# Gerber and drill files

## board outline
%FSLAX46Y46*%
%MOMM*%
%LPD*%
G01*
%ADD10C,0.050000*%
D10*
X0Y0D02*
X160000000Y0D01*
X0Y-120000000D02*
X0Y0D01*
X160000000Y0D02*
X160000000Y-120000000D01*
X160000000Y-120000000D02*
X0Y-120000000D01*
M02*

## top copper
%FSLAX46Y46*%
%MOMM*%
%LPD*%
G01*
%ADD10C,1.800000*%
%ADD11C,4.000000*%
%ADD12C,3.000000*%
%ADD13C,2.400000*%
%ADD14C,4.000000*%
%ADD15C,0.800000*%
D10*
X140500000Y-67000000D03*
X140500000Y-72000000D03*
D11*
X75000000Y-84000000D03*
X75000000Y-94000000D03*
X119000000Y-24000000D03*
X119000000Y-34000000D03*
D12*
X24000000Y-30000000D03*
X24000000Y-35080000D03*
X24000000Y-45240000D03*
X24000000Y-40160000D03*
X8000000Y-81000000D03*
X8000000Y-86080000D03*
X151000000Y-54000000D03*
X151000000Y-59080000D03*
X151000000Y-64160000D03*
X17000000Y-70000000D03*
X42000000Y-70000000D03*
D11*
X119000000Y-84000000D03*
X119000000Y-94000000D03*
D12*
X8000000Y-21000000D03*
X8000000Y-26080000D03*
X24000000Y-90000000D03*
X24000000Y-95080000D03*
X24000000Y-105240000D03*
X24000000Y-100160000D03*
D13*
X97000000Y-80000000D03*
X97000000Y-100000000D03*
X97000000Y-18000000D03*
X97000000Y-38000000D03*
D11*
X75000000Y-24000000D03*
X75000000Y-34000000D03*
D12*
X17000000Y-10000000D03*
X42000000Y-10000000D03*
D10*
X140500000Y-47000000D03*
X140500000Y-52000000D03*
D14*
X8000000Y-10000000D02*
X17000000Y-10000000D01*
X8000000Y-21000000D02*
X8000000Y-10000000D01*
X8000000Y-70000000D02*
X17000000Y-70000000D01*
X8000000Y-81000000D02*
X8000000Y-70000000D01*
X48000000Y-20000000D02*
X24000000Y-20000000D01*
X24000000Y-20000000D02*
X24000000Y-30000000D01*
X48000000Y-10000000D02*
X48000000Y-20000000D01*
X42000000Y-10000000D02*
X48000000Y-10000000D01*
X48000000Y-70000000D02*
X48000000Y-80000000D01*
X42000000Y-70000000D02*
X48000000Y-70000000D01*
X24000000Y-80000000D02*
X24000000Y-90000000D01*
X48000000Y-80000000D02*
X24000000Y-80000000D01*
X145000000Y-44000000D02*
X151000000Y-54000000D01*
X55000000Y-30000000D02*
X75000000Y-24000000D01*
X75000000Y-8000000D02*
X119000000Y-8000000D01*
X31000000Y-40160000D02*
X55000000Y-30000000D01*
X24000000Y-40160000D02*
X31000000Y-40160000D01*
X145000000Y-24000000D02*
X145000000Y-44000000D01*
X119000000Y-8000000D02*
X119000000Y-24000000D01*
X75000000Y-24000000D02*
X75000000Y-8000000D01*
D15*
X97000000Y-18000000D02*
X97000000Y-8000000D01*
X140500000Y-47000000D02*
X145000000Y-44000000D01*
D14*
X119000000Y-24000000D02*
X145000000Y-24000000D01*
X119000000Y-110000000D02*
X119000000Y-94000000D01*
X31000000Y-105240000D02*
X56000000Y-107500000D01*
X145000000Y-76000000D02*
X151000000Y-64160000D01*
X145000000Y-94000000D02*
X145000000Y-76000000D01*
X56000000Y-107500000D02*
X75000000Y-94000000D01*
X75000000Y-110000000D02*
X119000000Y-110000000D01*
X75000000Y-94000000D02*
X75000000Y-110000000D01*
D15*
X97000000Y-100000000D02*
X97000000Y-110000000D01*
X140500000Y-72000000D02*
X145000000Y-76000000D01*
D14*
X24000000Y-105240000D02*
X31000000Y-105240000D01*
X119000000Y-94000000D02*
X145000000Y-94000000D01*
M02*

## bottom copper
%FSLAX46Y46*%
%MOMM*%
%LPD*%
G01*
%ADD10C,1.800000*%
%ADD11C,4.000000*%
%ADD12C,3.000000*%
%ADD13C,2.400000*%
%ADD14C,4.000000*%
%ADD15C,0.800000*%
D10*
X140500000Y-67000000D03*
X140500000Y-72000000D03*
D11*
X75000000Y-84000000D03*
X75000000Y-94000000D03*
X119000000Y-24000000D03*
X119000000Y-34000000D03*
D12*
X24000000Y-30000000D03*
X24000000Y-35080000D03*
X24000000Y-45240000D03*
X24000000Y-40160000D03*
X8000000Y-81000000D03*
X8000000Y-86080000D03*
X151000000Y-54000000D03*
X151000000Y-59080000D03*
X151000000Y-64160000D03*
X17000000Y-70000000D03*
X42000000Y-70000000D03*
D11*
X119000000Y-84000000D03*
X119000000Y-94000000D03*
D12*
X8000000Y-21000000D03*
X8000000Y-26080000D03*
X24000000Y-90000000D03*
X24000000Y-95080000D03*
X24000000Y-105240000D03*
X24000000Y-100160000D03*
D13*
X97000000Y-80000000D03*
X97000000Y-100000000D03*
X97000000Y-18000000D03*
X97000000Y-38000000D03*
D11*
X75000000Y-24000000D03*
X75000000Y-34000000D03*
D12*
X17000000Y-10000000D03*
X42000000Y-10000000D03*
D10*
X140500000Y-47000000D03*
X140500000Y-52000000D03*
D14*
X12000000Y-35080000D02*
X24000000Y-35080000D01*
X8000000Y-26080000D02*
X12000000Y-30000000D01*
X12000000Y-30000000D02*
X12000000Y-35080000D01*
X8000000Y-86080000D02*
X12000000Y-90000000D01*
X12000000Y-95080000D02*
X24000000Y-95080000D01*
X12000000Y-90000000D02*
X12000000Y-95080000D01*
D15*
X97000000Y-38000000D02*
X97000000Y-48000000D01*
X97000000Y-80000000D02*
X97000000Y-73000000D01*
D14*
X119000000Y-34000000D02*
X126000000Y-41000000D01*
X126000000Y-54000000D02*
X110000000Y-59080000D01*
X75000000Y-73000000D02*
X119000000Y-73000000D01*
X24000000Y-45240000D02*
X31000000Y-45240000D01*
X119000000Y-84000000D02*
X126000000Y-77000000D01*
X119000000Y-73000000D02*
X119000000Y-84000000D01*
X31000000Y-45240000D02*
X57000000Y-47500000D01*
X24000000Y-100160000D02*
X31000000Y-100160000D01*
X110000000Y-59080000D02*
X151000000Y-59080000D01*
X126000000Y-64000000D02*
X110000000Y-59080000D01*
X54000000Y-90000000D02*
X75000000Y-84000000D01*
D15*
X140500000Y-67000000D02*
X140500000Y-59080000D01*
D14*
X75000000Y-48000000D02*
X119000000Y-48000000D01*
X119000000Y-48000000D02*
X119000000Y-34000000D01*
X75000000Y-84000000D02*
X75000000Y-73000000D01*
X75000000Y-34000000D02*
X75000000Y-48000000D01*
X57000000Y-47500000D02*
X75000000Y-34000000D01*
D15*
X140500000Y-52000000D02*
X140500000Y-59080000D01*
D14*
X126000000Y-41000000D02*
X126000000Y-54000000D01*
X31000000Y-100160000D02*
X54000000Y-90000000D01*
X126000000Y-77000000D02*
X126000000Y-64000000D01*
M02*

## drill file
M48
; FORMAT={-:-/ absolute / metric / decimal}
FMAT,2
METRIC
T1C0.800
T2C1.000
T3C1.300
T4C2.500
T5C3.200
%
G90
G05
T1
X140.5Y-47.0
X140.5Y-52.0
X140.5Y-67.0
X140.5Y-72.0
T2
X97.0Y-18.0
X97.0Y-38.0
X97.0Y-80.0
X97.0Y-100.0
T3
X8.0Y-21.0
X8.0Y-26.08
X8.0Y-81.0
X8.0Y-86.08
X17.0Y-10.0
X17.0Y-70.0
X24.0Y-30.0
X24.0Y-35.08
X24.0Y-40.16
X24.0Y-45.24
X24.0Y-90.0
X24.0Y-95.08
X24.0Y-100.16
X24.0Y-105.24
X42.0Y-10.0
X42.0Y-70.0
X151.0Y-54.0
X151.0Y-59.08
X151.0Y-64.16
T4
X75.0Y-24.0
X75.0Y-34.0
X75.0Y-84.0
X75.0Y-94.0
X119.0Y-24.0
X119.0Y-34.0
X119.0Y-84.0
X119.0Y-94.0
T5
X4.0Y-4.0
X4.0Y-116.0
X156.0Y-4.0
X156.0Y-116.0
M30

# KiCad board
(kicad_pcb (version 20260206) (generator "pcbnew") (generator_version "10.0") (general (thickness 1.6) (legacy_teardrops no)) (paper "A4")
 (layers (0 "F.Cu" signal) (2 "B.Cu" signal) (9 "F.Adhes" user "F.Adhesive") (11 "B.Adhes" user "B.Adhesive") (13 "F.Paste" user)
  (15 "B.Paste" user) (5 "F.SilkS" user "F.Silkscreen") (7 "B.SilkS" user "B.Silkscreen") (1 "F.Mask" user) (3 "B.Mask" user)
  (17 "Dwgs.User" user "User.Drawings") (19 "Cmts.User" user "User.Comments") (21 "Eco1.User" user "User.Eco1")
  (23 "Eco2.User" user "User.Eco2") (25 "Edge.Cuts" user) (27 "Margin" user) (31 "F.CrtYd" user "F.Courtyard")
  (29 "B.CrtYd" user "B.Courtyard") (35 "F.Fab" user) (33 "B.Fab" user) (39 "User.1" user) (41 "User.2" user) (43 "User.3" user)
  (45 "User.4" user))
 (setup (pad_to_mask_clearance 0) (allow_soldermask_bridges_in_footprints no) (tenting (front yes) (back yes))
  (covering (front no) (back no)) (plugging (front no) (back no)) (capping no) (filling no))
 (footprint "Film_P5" (layer "F.Cu") (at 140.5 67 -90)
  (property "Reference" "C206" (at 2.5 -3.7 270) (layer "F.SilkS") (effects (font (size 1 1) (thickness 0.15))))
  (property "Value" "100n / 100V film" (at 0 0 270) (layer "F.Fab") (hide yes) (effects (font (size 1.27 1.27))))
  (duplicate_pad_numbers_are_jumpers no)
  (pad "1" thru_hole circle (at 0 0 270) (size 1.8 1.8) (drill 0.8) (layers "*.Cu" "*.Mask") (remove_unused_layers no) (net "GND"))
  (pad "2" thru_hole circle (at 5 0 270) (size 1.8 1.8) (drill 0.8) (layers "*.Cu" "*.Mask") (remove_unused_layers no) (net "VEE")))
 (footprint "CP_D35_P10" (layer "F.Cu") (at 75 84 -90)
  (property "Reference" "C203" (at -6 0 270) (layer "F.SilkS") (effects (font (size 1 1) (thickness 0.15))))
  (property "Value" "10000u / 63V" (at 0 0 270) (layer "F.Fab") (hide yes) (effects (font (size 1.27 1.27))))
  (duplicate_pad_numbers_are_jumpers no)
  (pad "1" thru_hole circle (at 0 0 270) (size 4 4) (drill 2.5) (layers "*.Cu" "*.Mask") (remove_unused_layers no) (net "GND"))
  (pad "2" thru_hole circle (at 10 0 270) (size 4 4) (drill 2.5) (layers "*.Cu" "*.Mask") (remove_unused_layers no) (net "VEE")))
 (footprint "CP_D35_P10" (layer "F.Cu") (at 119 24 -90)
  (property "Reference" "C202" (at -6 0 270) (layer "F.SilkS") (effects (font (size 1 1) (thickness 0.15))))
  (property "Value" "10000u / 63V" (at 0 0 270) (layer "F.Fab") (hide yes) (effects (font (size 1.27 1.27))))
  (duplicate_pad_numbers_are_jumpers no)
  (pad "1" thru_hole circle (at 0 0 270) (size 4 4) (drill 2.5) (layers "*.Cu" "*.Mask") (remove_unused_layers no) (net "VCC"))
  (pad "2" thru_hole circle (at 10 0 270) (size 4 4) (drill 2.5) (layers "*.Cu" "*.Mask") (remove_unused_layers no) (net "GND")))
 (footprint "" (layer "F.Cu") (at 156 116)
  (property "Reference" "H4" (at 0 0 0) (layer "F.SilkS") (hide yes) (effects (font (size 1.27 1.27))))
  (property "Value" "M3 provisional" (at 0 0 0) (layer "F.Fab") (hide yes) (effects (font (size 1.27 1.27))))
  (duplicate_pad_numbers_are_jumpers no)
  (pad "" np_thru_hole circle (at 0 0) (size 3.2 3.2) (drill 3.2) (layers "*.Cu" "*.Mask")))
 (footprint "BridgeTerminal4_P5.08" (layer "F.Cu") (at 24 30 -90)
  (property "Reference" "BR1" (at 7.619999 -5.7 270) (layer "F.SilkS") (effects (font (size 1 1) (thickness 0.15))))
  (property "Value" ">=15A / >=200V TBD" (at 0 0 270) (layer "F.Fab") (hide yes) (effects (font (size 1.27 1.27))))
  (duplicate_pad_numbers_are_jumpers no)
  (pad "AC1" thru_hole circle (at 0 0 270) (size 3 3) (drill 1.3) (layers "*.Cu" "*.Mask") (remove_unused_layers no) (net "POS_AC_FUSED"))
  (pad "AC2" thru_hole circle (at 5.08 0 270) (size 3 3) (drill 1.3) (layers "*.Cu" "*.Mask") (remove_unused_layers no) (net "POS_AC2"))
  (pad "N" thru_hole circle (at 15.24 0 270) (size 3 3) (drill 1.3) (layers "*.Cu" "*.Mask") (remove_unused_layers no) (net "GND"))
  (pad "P" thru_hole circle (at 10.16 0 270) (size 3 3) (drill 1.3) (layers "*.Cu" "*.Mask") (remove_unused_layers no) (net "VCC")))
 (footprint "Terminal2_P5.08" (layer "F.Cu") (at 8 81 -90)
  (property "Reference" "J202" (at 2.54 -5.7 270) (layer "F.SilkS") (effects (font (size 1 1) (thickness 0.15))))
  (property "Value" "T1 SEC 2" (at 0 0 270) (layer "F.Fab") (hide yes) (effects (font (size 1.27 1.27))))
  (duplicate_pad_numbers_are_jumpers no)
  (pad "1" thru_hole circle (at 0 0 270) (size 3 3) (drill 1.3) (layers "*.Cu" "*.Mask") (remove_unused_layers no) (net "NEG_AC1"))
  (pad "2" thru_hole circle (at 5.08 0 270) (size 3 3) (drill 1.3) (layers "*.Cu" "*.Mask") (remove_unused_layers no) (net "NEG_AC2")))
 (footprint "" (layer "F.Cu") (at 4 4)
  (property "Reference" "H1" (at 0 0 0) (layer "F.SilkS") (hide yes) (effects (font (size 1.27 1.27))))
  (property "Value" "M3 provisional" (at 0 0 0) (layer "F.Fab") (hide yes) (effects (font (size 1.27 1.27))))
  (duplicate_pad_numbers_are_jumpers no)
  (pad "" np_thru_hole circle (at 0 0) (size 3.2 3.2) (drill 3.2) (layers "*.Cu" "*.Mask")))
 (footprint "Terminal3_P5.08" (layer "F.Cu") (at 151 54 -90)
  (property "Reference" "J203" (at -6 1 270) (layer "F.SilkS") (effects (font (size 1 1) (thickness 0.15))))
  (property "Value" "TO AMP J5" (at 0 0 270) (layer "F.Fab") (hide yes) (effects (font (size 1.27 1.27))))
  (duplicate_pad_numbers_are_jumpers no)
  (pad "1" thru_hole circle (at 0 0 270) (size 3 3) (drill 1.3) (layers "*.Cu" "*.Mask") (remove_unused_layers no) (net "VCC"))
  (pad "2" thru_hole circle (at 5.08 0 270) (size 3 3) (drill 1.3) (layers "*.Cu" "*.Mask") (remove_unused_layers no) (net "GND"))
  (pad "3" thru_hole circle (at 10.16 0 270) (size 3 3) (drill 1.3) (layers "*.Cu" "*.Mask") (remove_unused_layers no) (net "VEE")))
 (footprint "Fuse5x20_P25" (layer "F.Cu") (at 17 70)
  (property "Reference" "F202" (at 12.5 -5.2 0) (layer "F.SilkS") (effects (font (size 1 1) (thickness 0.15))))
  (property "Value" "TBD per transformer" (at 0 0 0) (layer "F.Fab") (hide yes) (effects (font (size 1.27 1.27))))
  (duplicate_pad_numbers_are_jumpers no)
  (pad "1" thru_hole circle (at 0 0) (size 3 3) (drill 1.3) (layers "*.Cu" "*.Mask") (remove_unused_layers no) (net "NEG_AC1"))
  (pad "2" thru_hole circle (at 25 0) (size 3 3) (drill 1.3) (layers "*.Cu" "*.Mask") (remove_unused_layers no) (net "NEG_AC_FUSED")))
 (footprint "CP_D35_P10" (layer "F.Cu") (at 119 84 -90)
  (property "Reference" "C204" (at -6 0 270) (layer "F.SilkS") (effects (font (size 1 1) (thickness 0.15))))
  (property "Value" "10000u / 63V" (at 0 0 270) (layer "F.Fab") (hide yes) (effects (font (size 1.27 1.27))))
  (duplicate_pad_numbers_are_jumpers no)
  (pad "1" thru_hole circle (at 0 0 270) (size 4 4) (drill 2.5) (layers "*.Cu" "*.Mask") (remove_unused_layers no) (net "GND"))
  (pad "2" thru_hole circle (at 10 0 270) (size 4 4) (drill 2.5) (layers "*.Cu" "*.Mask") (remove_unused_layers no) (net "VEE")))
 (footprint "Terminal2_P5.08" (layer "F.Cu") (at 8 21 -90)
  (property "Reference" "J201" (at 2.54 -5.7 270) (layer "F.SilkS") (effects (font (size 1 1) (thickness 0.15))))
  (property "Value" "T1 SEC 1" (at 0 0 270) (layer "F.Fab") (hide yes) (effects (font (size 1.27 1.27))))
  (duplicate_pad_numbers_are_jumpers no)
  (pad "1" thru_hole circle (at 0 0 270) (size 3 3) (drill 1.3) (layers "*.Cu" "*.Mask") (remove_unused_layers no) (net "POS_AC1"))
  (pad "2" thru_hole circle (at 5.08 0 270) (size 3 3) (drill 1.3) (layers "*.Cu" "*.Mask") (remove_unused_layers no) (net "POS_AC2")))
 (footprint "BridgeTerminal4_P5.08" (layer "F.Cu") (at 24 90 -90)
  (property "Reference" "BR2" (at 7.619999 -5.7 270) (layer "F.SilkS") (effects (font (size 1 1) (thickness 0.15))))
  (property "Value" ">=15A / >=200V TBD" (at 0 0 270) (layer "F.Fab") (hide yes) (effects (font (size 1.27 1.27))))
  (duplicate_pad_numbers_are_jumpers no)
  (pad "AC1" thru_hole circle (at 0 0 270) (size 3 3) (drill 1.3) (layers "*.Cu" "*.Mask") (remove_unused_layers no) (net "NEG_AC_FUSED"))
  (pad "AC2" thru_hole circle (at 5.08 0 270) (size 3 3) (drill 1.3) (layers "*.Cu" "*.Mask") (remove_unused_layers no) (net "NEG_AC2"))
  (pad "N" thru_hole circle (at 15.24 0 270) (size 3 3) (drill 1.3) (layers "*.Cu" "*.Mask") (remove_unused_layers no) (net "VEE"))
  (pad "P" thru_hole circle (at 10.16 0 270) (size 3 3) (drill 1.3) (layers "*.Cu" "*.Mask") (remove_unused_layers no) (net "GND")))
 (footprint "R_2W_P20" (layer "F.Cu") (at 97 80 -90)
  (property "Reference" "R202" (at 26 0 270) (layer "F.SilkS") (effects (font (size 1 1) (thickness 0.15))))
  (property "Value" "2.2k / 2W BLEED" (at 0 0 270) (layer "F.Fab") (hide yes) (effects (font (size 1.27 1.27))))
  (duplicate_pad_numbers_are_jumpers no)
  (pad "1" thru_hole circle (at 0 0 270) (size 2.4 2.4) (drill 1) (layers "*.Cu" "*.Mask") (remove_unused_layers no) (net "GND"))
  (pad "2" thru_hole circle (at 20 0 270) (size 2.4 2.4) (drill 1) (layers "*.Cu" "*.Mask") (remove_unused_layers no) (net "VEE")))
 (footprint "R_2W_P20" (layer "F.Cu") (at 97 18 -90)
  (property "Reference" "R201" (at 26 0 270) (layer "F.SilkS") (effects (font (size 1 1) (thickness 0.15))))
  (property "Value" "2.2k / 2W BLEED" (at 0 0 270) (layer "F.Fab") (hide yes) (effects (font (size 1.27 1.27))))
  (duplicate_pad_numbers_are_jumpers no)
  (pad "1" thru_hole circle (at 0 0 270) (size 2.4 2.4) (drill 1) (layers "*.Cu" "*.Mask") (remove_unused_layers no) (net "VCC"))
  (pad "2" thru_hole circle (at 20 0 270) (size 2.4 2.4) (drill 1) (layers "*.Cu" "*.Mask") (remove_unused_layers no) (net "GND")))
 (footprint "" (layer "F.Cu") (at 156 4)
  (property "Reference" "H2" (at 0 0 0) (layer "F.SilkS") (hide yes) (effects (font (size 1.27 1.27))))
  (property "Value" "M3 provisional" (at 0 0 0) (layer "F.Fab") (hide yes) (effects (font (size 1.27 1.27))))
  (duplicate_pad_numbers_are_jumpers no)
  (pad "" np_thru_hole circle (at 0 0) (size 3.2 3.2) (drill 3.2) (layers "*.Cu" "*.Mask")))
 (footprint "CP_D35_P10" (layer "F.Cu") (at 75 24 -90)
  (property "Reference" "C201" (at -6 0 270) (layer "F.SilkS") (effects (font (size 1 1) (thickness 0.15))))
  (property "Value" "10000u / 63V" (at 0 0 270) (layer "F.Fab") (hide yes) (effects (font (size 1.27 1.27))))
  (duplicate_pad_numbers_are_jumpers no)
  (pad "1" thru_hole circle (at 0 0 270) (size 4 4) (drill 2.5) (layers "*.Cu" "*.Mask") (remove_unused_layers no) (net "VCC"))
  (pad "2" thru_hole circle (at 10 0 270) (size 4 4) (drill 2.5) (layers "*.Cu" "*.Mask") (remove_unused_layers no) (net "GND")))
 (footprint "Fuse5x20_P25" (layer "F.Cu") (at 17 10)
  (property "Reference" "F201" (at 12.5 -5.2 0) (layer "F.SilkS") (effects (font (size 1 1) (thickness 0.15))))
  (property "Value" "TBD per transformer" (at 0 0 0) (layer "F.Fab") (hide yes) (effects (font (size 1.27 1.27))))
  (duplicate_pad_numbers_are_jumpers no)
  (pad "1" thru_hole circle (at 0 0) (size 3 3) (drill 1.3) (layers "*.Cu" "*.Mask") (remove_unused_layers no) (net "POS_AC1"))
  (pad "2" thru_hole circle (at 25 0) (size 3 3) (drill 1.3) (layers "*.Cu" "*.Mask") (remove_unused_layers no) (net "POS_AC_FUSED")))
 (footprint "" (layer "F.Cu") (at 4 116)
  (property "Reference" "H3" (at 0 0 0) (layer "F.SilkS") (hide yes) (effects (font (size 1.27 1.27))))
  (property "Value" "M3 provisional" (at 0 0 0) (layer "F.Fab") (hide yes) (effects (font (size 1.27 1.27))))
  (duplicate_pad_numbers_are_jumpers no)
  (pad "" np_thru_hole circle (at 0 0) (size 3.2 3.2) (drill 3.2) (layers "*.Cu" "*.Mask")))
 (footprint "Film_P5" (layer "F.Cu") (at 140.5 47 -90)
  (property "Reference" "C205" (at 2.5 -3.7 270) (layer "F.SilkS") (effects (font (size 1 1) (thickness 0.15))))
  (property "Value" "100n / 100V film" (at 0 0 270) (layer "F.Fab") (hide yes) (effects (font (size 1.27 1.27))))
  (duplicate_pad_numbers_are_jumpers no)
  (pad "1" thru_hole circle (at 0 0 270) (size 1.8 1.8) (drill 0.8) (layers "*.Cu" "*.Mask") (remove_unused_layers no) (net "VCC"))
  (pad "2" thru_hole circle (at 5 0 270) (size 1.8 1.8) (drill 0.8) (layers "*.Cu" "*.Mask") (remove_unused_layers no) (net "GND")))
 (gr_line (start 0 0) (end 160 0) (stroke (width 0.05) (type default)) (layer "Edge.Cuts"))
 (gr_line (start 0 120) (end 0 0) (stroke (width 0.05) (type default)) (layer "Edge.Cuts"))
 (gr_line (start 160 0) (end 160 120) (stroke (width 0.05) (type default)) (layer "Edge.Cuts"))
 (gr_line (start 160 120) (end 0 120) (stroke (width 0.05) (type default)) (layer "Edge.Cuts"))
 (segment (start 8 10) (end 17 10) (width 4) (layer "F.Cu") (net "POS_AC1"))
 (segment (start 8 21) (end 8 10) (width 4) (layer "F.Cu") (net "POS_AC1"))
 (segment (start 12 35.08) (end 24 35.08) (width 4) (layer "B.Cu") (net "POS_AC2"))
 (segment (start 8 26.08) (end 12 30) (width 4) (layer "B.Cu") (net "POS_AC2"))
 (segment (start 12 30) (end 12 35.08) (width 4) (layer "B.Cu") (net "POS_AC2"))
 (segment (start 8 70) (end 17 70) (width 4) (layer "F.Cu") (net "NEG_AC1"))
 (segment (start 8 81) (end 8 70) (width 4) (layer "F.Cu") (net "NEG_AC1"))
 (segment (start 8 86.08) (end 12 90) (width 4) (layer "B.Cu") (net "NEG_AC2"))
 (segment (start 12 95.08) (end 24 95.08) (width 4) (layer "B.Cu") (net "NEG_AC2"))
 (segment (start 12 90) (end 12 95.08) (width 4) (layer "B.Cu") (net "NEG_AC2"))
 (segment (start 48 20) (end 24 20) (width 4) (layer "F.Cu") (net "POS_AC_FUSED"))
 (segment (start 24 20) (end 24 30) (width 4) (layer "F.Cu") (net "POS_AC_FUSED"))
 (segment (start 48 10) (end 48 20) (width 4) (layer "F.Cu") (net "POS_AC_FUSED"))
 (segment (start 42 10) (end 48 10) (width 4) (layer "F.Cu") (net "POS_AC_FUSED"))
 (segment (start 48 70) (end 48 80) (width 4) (layer "F.Cu") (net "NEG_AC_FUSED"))
 (segment (start 42 70) (end 48 70) (width 4) (layer "F.Cu") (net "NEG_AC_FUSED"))
 (segment (start 24 80) (end 24 90) (width 4) (layer "F.Cu") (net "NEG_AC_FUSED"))
 (segment (start 48 80) (end 24 80) (width 4) (layer "F.Cu") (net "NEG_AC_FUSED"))
 (segment (start 97 38) (end 97 48) (width 0.8) (layer "B.Cu") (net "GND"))
 (segment (start 97 80) (end 97 73) (width 0.8) (layer "B.Cu") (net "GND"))
 (segment (start 119 34) (end 126 41) (width 4) (layer "B.Cu") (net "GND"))
 (segment (start 126 54) (end 110 59.08) (width 4) (layer "B.Cu") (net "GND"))
 (segment (start 75 73) (end 119 73) (width 4) (layer "B.Cu") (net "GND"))
 (segment (start 24 45.24) (end 31 45.24) (width 4) (layer "B.Cu") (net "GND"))
 (segment (start 119 84) (end 126 77) (width 4) (layer "B.Cu") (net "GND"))
 (segment (start 119 73) (end 119 84) (width 4) (layer "B.Cu") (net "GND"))
 (segment (start 31 45.24) (end 57 47.5) (width 4) (layer "B.Cu") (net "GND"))
 (segment (start 24 100.16) (end 31 100.16) (width 4) (layer "B.Cu") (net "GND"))
 (segment (start 110 59.08) (end 151 59.08) (width 4) (layer "B.Cu") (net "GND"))
 (segment (start 126 64) (end 110 59.08) (width 4) (layer "B.Cu") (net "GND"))
 (segment (start 54 90) (end 75 84) (width 4) (layer "B.Cu") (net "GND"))
 (segment (start 140.5 67) (end 140.5 59.08) (width 0.8) (layer "B.Cu") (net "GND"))
 (segment (start 75 48) (end 119 48) (width 4) (layer "B.Cu") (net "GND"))
 (segment (start 119 48) (end 119 34) (width 4) (layer "B.Cu") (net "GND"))
 (segment (start 75 84) (end 75 73) (width 4) (layer "B.Cu") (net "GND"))
 (segment (start 75 34) (end 75 48) (width 4) (layer "B.Cu") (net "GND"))
 (segment (start 57 47.5) (end 75 34) (width 4) (layer "B.Cu") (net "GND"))
 (segment (start 140.5 52) (end 140.5 59.08) (width 0.8) (layer "B.Cu") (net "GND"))
 (segment (start 126 41) (end 126 54) (width 4) (layer "B.Cu") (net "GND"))
 (segment (start 31 100.16) (end 54 90) (width 4) (layer "B.Cu") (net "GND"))
 (segment (start 126 77) (end 126 64) (width 4) (layer "B.Cu") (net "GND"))
 (segment (start 145 44) (end 151 54) (width 4) (layer "F.Cu") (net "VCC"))
 (segment (start 55 30) (end 75 24) (width 4) (layer "F.Cu") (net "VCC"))
 (segment (start 75 8) (end 119 8) (width 4) (layer "F.Cu") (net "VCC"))
 (segment (start 31 40.16) (end 55 30) (width 4) (layer "F.Cu") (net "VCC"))
 (segment (start 24 40.16) (end 31 40.16) (width 4) (layer "F.Cu") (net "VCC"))
 (segment (start 145 24) (end 145 44) (width 4) (layer "F.Cu") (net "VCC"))
 (segment (start 119 8) (end 119 24) (width 4) (layer "F.Cu") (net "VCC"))
 (segment (start 75 24) (end 75 8) (width 4) (layer "F.Cu") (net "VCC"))
 (segment (start 97 18) (end 97 8) (width 0.8) (layer "F.Cu") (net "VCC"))
 (segment (start 140.5 47) (end 145 44) (width 0.8) (layer "F.Cu") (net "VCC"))
 (segment (start 119 24) (end 145 24) (width 4) (layer "F.Cu") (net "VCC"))
 (segment (start 119 110) (end 119 94) (width 4) (layer "F.Cu") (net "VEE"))
 (segment (start 31 105.24) (end 56 107.5) (width 4) (layer "F.Cu") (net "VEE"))
 (segment (start 145 76) (end 151 64.16) (width 4) (layer "F.Cu") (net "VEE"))
 (segment (start 145 94) (end 145 76) (width 4) (layer "F.Cu") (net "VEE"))
 (segment (start 56 107.5) (end 75 94) (width 4) (layer "F.Cu") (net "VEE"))
 (segment (start 75 110) (end 119 110) (width 4) (layer "F.Cu") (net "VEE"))
 (segment (start 75 94) (end 75 110) (width 4) (layer "F.Cu") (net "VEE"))
 (segment (start 97 100) (end 97 110) (width 0.8) (layer "F.Cu") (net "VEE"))
 (segment (start 140.5 72) (end 145 76) (width 0.8) (layer "F.Cu") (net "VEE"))
 (segment (start 24 105.24) (end 31 105.24) (width 4) (layer "F.Cu") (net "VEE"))
 (segment (start 119 94) (end 145 94) (width 4) (layer "F.Cu") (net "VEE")))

